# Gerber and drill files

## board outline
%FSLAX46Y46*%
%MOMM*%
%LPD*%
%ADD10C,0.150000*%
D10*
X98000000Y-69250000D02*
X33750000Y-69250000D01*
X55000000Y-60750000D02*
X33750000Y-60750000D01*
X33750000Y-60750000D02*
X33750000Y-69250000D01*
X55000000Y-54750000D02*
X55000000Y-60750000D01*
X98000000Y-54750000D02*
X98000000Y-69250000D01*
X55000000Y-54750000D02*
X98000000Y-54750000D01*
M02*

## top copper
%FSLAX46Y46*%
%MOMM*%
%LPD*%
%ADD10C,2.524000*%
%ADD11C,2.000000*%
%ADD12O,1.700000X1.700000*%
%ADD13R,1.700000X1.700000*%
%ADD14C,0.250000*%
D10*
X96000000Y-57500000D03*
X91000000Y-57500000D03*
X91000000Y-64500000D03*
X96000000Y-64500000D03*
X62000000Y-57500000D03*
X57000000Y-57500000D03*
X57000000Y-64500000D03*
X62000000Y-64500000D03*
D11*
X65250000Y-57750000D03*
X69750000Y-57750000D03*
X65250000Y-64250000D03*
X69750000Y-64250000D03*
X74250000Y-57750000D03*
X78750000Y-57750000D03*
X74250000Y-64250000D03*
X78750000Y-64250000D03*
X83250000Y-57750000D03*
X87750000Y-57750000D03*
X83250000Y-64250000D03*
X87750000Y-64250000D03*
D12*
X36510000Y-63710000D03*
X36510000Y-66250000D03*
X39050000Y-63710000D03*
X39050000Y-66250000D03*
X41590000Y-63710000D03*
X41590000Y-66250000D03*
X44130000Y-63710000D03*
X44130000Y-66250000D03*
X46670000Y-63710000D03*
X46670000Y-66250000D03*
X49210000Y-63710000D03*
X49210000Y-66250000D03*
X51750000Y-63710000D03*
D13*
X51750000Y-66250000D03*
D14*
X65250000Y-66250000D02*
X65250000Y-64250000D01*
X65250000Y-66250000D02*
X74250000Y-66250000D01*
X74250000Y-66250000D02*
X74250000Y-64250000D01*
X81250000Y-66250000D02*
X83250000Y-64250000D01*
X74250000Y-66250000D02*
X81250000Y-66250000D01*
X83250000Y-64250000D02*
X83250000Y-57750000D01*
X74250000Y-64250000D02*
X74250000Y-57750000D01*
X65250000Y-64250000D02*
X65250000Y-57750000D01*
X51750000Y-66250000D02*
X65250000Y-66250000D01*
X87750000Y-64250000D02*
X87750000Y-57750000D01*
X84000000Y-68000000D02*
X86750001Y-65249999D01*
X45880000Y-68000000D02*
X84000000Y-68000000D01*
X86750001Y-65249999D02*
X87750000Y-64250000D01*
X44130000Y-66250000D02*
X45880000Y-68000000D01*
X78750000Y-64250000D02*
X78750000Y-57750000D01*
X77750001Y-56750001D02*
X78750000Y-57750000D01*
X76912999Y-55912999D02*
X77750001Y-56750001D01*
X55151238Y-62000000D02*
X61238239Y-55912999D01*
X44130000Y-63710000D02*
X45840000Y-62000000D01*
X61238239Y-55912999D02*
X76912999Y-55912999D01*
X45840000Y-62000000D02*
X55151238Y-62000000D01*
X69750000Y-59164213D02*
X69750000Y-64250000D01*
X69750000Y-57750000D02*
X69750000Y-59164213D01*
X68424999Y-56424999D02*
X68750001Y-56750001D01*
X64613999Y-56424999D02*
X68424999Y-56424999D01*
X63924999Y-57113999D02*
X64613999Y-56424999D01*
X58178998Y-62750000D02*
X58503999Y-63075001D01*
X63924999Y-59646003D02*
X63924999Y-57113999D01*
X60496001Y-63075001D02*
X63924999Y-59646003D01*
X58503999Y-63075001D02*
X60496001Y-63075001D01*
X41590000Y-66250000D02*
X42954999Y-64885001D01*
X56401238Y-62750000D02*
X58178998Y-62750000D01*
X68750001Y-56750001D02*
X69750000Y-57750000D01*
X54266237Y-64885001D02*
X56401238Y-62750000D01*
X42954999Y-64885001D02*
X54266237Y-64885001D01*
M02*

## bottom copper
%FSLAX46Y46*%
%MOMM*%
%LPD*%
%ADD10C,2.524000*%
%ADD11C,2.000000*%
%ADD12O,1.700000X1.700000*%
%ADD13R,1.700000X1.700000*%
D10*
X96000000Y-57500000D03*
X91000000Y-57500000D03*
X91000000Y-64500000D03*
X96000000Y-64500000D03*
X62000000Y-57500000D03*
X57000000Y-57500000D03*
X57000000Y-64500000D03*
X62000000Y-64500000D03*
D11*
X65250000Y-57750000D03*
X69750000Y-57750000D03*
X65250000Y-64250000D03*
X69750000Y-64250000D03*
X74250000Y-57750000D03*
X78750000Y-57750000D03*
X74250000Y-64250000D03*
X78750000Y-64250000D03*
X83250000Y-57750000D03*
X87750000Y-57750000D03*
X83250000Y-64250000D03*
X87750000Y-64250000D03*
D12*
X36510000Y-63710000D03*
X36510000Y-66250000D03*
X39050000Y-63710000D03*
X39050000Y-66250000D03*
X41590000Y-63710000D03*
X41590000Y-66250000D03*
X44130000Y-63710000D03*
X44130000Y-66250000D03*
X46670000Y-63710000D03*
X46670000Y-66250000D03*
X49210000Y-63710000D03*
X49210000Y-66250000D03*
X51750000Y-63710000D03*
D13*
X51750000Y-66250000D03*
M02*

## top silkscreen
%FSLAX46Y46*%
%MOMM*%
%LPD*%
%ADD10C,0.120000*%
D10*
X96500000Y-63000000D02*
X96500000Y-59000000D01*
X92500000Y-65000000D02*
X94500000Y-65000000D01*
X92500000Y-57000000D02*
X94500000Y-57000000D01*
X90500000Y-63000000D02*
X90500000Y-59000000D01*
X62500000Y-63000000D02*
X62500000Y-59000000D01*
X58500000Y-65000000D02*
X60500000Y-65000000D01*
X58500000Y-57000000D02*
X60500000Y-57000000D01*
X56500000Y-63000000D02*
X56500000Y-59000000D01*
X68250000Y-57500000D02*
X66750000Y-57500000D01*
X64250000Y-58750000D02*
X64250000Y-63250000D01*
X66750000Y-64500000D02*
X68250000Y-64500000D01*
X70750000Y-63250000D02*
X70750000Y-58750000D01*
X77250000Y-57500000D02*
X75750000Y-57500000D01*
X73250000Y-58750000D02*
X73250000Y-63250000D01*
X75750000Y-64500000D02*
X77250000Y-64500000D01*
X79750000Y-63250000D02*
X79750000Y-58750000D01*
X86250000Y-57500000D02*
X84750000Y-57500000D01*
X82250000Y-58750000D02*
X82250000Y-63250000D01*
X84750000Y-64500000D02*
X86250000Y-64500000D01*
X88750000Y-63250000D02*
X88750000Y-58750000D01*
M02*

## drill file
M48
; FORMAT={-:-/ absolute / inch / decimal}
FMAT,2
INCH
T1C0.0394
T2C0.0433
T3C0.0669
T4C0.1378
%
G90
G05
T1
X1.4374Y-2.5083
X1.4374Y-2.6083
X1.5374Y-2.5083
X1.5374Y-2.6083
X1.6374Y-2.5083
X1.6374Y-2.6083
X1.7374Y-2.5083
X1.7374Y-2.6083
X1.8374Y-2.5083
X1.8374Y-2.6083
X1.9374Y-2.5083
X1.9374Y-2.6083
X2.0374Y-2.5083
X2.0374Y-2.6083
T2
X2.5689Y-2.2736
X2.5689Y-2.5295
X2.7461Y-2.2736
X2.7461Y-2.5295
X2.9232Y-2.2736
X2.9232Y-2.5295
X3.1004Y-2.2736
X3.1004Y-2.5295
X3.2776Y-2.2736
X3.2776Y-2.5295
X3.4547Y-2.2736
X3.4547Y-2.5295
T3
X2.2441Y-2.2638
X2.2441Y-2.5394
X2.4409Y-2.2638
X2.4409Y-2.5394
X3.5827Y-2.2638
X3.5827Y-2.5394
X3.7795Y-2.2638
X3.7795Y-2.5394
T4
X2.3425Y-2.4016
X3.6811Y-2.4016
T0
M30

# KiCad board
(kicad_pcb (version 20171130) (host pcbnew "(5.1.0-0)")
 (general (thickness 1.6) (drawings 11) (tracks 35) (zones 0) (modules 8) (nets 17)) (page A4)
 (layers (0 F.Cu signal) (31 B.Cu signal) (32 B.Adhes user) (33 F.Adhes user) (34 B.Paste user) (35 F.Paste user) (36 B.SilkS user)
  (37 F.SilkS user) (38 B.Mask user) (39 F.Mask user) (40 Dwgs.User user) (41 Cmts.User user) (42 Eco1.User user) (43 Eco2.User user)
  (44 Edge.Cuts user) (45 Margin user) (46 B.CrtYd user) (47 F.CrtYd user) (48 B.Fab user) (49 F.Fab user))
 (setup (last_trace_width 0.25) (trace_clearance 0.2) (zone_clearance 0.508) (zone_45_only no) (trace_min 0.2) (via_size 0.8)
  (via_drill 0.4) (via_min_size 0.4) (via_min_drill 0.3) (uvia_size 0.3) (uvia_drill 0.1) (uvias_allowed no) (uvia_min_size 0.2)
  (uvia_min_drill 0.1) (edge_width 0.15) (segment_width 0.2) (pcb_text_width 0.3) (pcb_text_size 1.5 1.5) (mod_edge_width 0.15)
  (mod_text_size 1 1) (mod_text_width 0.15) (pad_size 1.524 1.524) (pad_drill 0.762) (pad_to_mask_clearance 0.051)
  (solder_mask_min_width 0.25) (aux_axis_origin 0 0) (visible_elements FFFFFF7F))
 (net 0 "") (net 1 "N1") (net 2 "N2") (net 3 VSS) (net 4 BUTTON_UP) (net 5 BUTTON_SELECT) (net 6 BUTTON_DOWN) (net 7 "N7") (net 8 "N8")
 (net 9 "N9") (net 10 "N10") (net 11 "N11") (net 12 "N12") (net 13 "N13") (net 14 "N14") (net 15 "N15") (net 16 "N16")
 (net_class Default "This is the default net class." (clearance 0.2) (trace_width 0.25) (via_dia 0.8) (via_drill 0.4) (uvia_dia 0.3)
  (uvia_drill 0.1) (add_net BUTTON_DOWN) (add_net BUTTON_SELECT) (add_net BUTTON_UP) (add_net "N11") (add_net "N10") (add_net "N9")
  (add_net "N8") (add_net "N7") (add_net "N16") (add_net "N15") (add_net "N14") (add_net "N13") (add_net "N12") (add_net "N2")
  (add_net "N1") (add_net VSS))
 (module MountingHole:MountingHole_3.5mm (layer F.Cu) (at 59.5 61)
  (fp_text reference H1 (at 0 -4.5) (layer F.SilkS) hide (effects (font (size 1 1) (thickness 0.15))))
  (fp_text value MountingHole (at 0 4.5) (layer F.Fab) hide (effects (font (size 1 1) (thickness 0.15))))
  (pad 1 np_thru_hole circle (at 0 0) (size 3.5 3.5) (drill 3.5) (layers *.Cu *.Mask)))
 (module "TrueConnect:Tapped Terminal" (layer F.Cu) (at 93.5 61 90)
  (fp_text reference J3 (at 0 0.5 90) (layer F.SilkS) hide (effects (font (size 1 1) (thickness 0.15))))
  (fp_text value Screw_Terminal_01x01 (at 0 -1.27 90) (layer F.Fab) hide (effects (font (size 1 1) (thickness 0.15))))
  (fp_line (start -2 3) (end 2 3) (layer F.SilkS) (width 0.12))
  (fp_line (start -4 -1) (end -4 1) (layer F.SilkS) (width 0.12))
  (fp_line (start 4 -1) (end 4 1) (layer F.SilkS) (width 0.12))
  (fp_line (start -2 -3) (end 2 -3) (layer F.SilkS) (width 0.12))
  (pad 1 thru_hole circle (at 3.5 2.5 90) (size 2.524 2.524) (drill 1.7) (layers *.Cu *.Mask) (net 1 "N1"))
  (pad 1 thru_hole circle (at 3.5 -2.5 90) (size 2.524 2.524) (drill 1.7) (layers *.Cu *.Mask) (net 1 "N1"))
  (pad 1 thru_hole circle (at -3.5 -2.5 90) (size 2.524 2.524) (drill 1.7) (layers *.Cu *.Mask) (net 1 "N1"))
  (pad 1 thru_hole circle (at -3.5 2.5 90) (size 2.524 2.524) (drill 1.7) (layers *.Cu *.Mask) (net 1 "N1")))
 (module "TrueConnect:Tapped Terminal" (layer F.Cu) (at 59.5 61 90)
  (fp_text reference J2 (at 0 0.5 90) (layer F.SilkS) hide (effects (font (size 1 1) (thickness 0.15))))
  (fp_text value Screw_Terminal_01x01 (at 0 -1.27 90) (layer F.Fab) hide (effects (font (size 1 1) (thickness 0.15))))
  (fp_line (start -2 3) (end 2 3) (layer F.SilkS) (width 0.12))
  (fp_line (start -4 -1) (end -4 1) (layer F.SilkS) (width 0.12))
  (fp_line (start 4 -1) (end 4 1) (layer F.SilkS) (width 0.12))
  (fp_line (start -2 -3) (end 2 -3) (layer F.SilkS) (width 0.12))
  (pad 1 thru_hole circle (at 3.5 2.5 90) (size 2.524 2.524) (drill 1.7) (layers *.Cu *.Mask) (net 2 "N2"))
  (pad 1 thru_hole circle (at 3.5 -2.5 90) (size 2.524 2.524) (drill 1.7) (layers *.Cu *.Mask) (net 2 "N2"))
  (pad 1 thru_hole circle (at -3.5 -2.5 90) (size 2.524 2.524) (drill 1.7) (layers *.Cu *.Mask) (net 2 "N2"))
  (pad 1 thru_hole circle (at -3.5 2.5 90) (size 2.524 2.524) (drill 1.7) (layers *.Cu *.Mask) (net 2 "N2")))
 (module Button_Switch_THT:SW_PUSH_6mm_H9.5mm (layer F.Cu) (at 65.25 64.25 90)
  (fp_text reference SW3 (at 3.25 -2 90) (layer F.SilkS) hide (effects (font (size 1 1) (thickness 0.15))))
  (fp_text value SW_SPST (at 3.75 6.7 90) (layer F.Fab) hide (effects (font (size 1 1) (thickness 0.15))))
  (fp_line (start 6.75 3) (end 6.75 1.5) (layer F.SilkS) (width 0.12))
  (fp_line (start 5.5 -1) (end 1 -1) (layer F.SilkS) (width 0.12))
  (fp_line (start -0.25 1.5) (end -0.25 3) (layer F.SilkS) (width 0.12))
  (fp_line (start 1 5.5) (end 5.5 5.5) (layer F.SilkS) (width 0.12))
  (pad 1 thru_hole circle (at 6.5 0 180) (size 2 2) (drill 1.1) (layers *.Cu *.Mask) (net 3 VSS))
  (pad 2 thru_hole circle (at 6.5 4.5 180) (size 2 2) (drill 1.1) (layers *.Cu *.Mask) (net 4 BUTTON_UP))
  (pad 1 thru_hole circle (at 0 0 180) (size 2 2) (drill 1.1) (layers *.Cu *.Mask) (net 3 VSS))
  (pad 2 thru_hole circle (at 0 4.5 180) (size 2 2) (drill 1.1) (layers *.Cu *.Mask) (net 4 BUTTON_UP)))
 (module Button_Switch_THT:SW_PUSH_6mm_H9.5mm (layer F.Cu) (at 74.25 64.25 90)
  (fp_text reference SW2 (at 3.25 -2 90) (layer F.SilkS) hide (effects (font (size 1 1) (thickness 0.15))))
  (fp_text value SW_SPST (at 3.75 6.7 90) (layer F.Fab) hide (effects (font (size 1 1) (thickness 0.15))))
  (fp_line (start 6.75 3) (end 6.75 1.5) (layer F.SilkS) (width 0.12))
  (fp_line (start 5.5 -1) (end 1 -1) (layer F.SilkS) (width 0.12))
  (fp_line (start -0.25 1.5) (end -0.25 3) (layer F.SilkS) (width 0.12))
  (fp_line (start 1 5.5) (end 5.5 5.5) (layer F.SilkS) (width 0.12))
  (pad 1 thru_hole circle (at 6.5 0 180) (size 2 2) (drill 1.1) (layers *.Cu *.Mask) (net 3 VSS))
  (pad 2 thru_hole circle (at 6.5 4.5 180) (size 2 2) (drill 1.1) (layers *.Cu *.Mask) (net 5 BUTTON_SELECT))
  (pad 1 thru_hole circle (at 0 0 180) (size 2 2) (drill 1.1) (layers *.Cu *.Mask) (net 3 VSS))
  (pad 2 thru_hole circle (at 0 4.5 180) (size 2 2) (drill 1.1) (layers *.Cu *.Mask) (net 5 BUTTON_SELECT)))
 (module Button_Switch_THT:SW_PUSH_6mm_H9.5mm (layer F.Cu) (at 83.25 64.25 90)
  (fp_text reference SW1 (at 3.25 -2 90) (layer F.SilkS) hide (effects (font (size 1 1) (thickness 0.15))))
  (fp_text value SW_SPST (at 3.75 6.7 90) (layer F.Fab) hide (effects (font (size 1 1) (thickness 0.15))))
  (fp_line (start 6.75 3) (end 6.75 1.5) (layer F.SilkS) (width 0.12))
  (fp_line (start 5.5 -1) (end 1 -1) (layer F.SilkS) (width 0.12))
  (fp_line (start -0.25 1.5) (end -0.25 3) (layer F.SilkS) (width 0.12))
  (fp_line (start 1 5.5) (end 5.5 5.5) (layer F.SilkS) (width 0.12))
  (pad 1 thru_hole circle (at 6.5 0 180) (size 2 2) (drill 1.1) (layers *.Cu *.Mask) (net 3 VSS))
  (pad 2 thru_hole circle (at 6.5 4.5 180) (size 2 2) (drill 1.1) (layers *.Cu *.Mask) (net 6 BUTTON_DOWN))
  (pad 1 thru_hole circle (at 0 0 180) (size 2 2) (drill 1.1) (layers *.Cu *.Mask) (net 3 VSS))
  (pad 2 thru_hole circle (at 0 4.5 180) (size 2 2) (drill 1.1) (layers *.Cu *.Mask) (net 6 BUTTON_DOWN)))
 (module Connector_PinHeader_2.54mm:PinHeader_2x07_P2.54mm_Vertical (layer B.Cu) (at 51.75 66.25 90)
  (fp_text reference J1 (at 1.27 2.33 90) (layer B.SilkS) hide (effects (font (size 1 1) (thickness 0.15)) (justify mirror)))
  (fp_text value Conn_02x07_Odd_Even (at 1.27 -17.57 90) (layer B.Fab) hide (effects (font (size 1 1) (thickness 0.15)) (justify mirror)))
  (pad 14 thru_hole oval (at 2.54 -15.24 90) (size 1.7 1.7) (drill 1) (layers *.Cu *.Mask) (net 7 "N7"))
  (pad 13 thru_hole oval (at 0 -15.24 90) (size 1.7 1.7) (drill 1) (layers *.Cu *.Mask) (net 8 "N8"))
  (pad 12 thru_hole oval (at 2.54 -12.7 90) (size 1.7 1.7) (drill 1) (layers *.Cu *.Mask) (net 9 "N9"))
  (pad 11 thru_hole oval (at 0 -12.7 90) (size 1.7 1.7) (drill 1) (layers *.Cu *.Mask) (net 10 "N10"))
  (pad 10 thru_hole oval (at 2.54 -10.16 90) (size 1.7 1.7) (drill 1) (layers *.Cu *.Mask) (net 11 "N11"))
  (pad 9 thru_hole oval (at 0 -10.16 90) (size 1.7 1.7) (drill 1) (layers *.Cu *.Mask) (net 4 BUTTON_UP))
  (pad 8 thru_hole oval (at 2.54 -7.62 90) (size 1.7 1.7) (drill 1) (layers *.Cu *.Mask) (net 5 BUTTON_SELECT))
  (pad 7 thru_hole oval (at 0 -7.62 90) (size 1.7 1.7) (drill 1) (layers *.Cu *.Mask) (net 6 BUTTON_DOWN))
  (pad 6 thru_hole oval (at 2.54 -5.08 90) (size 1.7 1.7) (drill 1) (layers *.Cu *.Mask) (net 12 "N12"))
  (pad 5 thru_hole oval (at 0 -5.08 90) (size 1.7 1.7) (drill 1) (layers *.Cu *.Mask) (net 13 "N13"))
  (pad 4 thru_hole oval (at 2.54 -2.54 90) (size 1.7 1.7) (drill 1) (layers *.Cu *.Mask) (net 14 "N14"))
  (pad 3 thru_hole oval (at 0 -2.54 90) (size 1.7 1.7) (drill 1) (layers *.Cu *.Mask) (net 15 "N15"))
  (pad 2 thru_hole oval (at 2.54 0 90) (size 1.7 1.7) (drill 1) (layers *.Cu *.Mask) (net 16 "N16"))
  (pad 1 thru_hole rect (at 0 0 90) (size 1.7 1.7) (drill 1) (layers *.Cu *.Mask) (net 3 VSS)))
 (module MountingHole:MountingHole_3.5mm (layer F.Cu) (at 93.5 61)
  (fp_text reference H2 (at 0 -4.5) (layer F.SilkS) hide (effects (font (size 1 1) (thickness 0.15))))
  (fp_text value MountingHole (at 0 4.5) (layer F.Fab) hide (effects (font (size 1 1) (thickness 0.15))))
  (pad 1 np_thru_hole circle (at 0 0) (size 3.5 3.5) (drill 3.5) (layers *.Cu *.Mask)))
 (gr_line (start 98 69.25) (end 33.75 69.25) (layer Edge.Cuts) (width 0.15))
 (gr_line (start 55 60.75) (end 33.75 60.75) (layer Edge.Cuts) (width 0.15))
 (gr_line (start 33.75 60.75) (end 33.75 69.25) (layer Edge.Cuts) (width 0.15))
 (gr_line (start 55 54.75) (end 55 60.75) (layer Edge.Cuts) (width 0.15))
 (gr_line (start 98 54.75) (end 98 69.25) (layer Edge.Cuts) (width 0.15))
 (gr_line (start 55 54.75) (end 98 54.75) (layer Edge.Cuts) (width 0.15))
 (segment (start 65.25 66.25) (end 65.25 64.25) (width 0.25) (layer F.Cu) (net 3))
 (segment (start 65.25 66.25) (end 74.25 66.25) (width 0.25) (layer F.Cu) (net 3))
 (segment (start 74.25 66.25) (end 74.25 64.25) (width 0.25) (layer F.Cu) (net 3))
 (segment (start 81.25 66.25) (end 83.25 64.25) (width 0.25) (layer F.Cu) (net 3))
 (segment (start 74.25 66.25) (end 81.25 66.25) (width 0.25) (layer F.Cu) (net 3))
 (segment (start 83.25 64.25) (end 83.25 57.75) (width 0.25) (layer F.Cu) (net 3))
 (segment (start 74.25 64.25) (end 74.25 57.75) (width 0.25) (layer F.Cu) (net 3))
 (segment (start 65.25 64.25) (end 65.25 57.75) (width 0.25) (layer F.Cu) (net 3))
 (segment (start 51.75 66.25) (end 65.25 66.25) (width 0.25) (layer F.Cu) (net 3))
 (segment (start 87.75 64.25) (end 87.75 57.75) (width 0.25) (layer F.Cu) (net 6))
 (segment (start 84 68) (end 86.750001 65.249999) (width 0.25) (layer F.Cu) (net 6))
 (segment (start 45.88 68) (end 84 68) (width 0.25) (layer F.Cu) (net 6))
 (segment (start 86.750001 65.249999) (end 87.75 64.25) (width 0.25) (layer F.Cu) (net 6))
 (segment (start 44.13 66.25) (end 45.88 68) (width 0.25) (layer F.Cu) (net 6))
 (segment (start 78.75 64.25) (end 78.75 57.75) (width 0.25) (layer F.Cu) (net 5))
 (segment (start 77.750001 56.750001) (end 78.75 57.75) (width 0.25) (layer F.Cu) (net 5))
 (segment (start 76.912999 55.912999) (end 77.750001 56.750001) (width 0.25) (layer F.Cu) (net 5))
 (segment (start 55.151238 62) (end 61.238239 55.912999) (width 0.25) (layer F.Cu) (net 5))
 (segment (start 44.13 63.71) (end 45.84 62) (width 0.25) (layer F.Cu) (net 5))
 (segment (start 61.238239 55.912999) (end 76.912999 55.912999) (width 0.25) (layer F.Cu) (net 5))
 (segment (start 45.84 62) (end 55.151238 62) (width 0.25) (layer F.Cu) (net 5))
 (segment (start 69.75 59.164213) (end 69.75 64.25) (width 0.25) (layer F.Cu) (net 4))
 (segment (start 69.75 57.75) (end 69.75 59.164213) (width 0.25) (layer F.Cu) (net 4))
 (segment (start 68.424999 56.424999) (end 68.750001 56.750001) (width 0.25) (layer F.Cu) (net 4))
 (segment (start 64.613999 56.424999) (end 68.424999 56.424999) (width 0.25) (layer F.Cu) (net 4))
 (segment (start 63.924999 57.113999) (end 64.613999 56.424999) (width 0.25) (layer F.Cu) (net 4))
 (segment (start 58.178998 62.75) (end 58.503999 63.075001) (width 0.25) (layer F.Cu) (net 4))
 (segment (start 63.924999 59.646003) (end 63.924999 57.113999) (width 0.25) (layer F.Cu) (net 4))
 (segment (start 60.496001 63.075001) (end 63.924999 59.646003) (width 0.25) (layer F.Cu) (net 4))
 (segment (start 58.503999 63.075001) (end 60.496001 63.075001) (width 0.25) (layer F.Cu) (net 4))
 (segment (start 41.59 66.25) (end 42.954999 64.885001) (width 0.25) (layer F.Cu) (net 4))
 (segment (start 56.401238 62.75) (end 58.178998 62.75) (width 0.25) (layer F.Cu) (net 4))
 (segment (start 68.750001 56.750001) (end 69.75 57.75) (width 0.25) (layer F.Cu) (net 4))
 (segment (start 54.266237 64.885001) (end 56.401238 62.75) (width 0.25) (layer F.Cu) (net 4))
 (segment (start 42.954999 64.885001) (end 54.266237 64.885001) (width 0.25) (layer F.Cu) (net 4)))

